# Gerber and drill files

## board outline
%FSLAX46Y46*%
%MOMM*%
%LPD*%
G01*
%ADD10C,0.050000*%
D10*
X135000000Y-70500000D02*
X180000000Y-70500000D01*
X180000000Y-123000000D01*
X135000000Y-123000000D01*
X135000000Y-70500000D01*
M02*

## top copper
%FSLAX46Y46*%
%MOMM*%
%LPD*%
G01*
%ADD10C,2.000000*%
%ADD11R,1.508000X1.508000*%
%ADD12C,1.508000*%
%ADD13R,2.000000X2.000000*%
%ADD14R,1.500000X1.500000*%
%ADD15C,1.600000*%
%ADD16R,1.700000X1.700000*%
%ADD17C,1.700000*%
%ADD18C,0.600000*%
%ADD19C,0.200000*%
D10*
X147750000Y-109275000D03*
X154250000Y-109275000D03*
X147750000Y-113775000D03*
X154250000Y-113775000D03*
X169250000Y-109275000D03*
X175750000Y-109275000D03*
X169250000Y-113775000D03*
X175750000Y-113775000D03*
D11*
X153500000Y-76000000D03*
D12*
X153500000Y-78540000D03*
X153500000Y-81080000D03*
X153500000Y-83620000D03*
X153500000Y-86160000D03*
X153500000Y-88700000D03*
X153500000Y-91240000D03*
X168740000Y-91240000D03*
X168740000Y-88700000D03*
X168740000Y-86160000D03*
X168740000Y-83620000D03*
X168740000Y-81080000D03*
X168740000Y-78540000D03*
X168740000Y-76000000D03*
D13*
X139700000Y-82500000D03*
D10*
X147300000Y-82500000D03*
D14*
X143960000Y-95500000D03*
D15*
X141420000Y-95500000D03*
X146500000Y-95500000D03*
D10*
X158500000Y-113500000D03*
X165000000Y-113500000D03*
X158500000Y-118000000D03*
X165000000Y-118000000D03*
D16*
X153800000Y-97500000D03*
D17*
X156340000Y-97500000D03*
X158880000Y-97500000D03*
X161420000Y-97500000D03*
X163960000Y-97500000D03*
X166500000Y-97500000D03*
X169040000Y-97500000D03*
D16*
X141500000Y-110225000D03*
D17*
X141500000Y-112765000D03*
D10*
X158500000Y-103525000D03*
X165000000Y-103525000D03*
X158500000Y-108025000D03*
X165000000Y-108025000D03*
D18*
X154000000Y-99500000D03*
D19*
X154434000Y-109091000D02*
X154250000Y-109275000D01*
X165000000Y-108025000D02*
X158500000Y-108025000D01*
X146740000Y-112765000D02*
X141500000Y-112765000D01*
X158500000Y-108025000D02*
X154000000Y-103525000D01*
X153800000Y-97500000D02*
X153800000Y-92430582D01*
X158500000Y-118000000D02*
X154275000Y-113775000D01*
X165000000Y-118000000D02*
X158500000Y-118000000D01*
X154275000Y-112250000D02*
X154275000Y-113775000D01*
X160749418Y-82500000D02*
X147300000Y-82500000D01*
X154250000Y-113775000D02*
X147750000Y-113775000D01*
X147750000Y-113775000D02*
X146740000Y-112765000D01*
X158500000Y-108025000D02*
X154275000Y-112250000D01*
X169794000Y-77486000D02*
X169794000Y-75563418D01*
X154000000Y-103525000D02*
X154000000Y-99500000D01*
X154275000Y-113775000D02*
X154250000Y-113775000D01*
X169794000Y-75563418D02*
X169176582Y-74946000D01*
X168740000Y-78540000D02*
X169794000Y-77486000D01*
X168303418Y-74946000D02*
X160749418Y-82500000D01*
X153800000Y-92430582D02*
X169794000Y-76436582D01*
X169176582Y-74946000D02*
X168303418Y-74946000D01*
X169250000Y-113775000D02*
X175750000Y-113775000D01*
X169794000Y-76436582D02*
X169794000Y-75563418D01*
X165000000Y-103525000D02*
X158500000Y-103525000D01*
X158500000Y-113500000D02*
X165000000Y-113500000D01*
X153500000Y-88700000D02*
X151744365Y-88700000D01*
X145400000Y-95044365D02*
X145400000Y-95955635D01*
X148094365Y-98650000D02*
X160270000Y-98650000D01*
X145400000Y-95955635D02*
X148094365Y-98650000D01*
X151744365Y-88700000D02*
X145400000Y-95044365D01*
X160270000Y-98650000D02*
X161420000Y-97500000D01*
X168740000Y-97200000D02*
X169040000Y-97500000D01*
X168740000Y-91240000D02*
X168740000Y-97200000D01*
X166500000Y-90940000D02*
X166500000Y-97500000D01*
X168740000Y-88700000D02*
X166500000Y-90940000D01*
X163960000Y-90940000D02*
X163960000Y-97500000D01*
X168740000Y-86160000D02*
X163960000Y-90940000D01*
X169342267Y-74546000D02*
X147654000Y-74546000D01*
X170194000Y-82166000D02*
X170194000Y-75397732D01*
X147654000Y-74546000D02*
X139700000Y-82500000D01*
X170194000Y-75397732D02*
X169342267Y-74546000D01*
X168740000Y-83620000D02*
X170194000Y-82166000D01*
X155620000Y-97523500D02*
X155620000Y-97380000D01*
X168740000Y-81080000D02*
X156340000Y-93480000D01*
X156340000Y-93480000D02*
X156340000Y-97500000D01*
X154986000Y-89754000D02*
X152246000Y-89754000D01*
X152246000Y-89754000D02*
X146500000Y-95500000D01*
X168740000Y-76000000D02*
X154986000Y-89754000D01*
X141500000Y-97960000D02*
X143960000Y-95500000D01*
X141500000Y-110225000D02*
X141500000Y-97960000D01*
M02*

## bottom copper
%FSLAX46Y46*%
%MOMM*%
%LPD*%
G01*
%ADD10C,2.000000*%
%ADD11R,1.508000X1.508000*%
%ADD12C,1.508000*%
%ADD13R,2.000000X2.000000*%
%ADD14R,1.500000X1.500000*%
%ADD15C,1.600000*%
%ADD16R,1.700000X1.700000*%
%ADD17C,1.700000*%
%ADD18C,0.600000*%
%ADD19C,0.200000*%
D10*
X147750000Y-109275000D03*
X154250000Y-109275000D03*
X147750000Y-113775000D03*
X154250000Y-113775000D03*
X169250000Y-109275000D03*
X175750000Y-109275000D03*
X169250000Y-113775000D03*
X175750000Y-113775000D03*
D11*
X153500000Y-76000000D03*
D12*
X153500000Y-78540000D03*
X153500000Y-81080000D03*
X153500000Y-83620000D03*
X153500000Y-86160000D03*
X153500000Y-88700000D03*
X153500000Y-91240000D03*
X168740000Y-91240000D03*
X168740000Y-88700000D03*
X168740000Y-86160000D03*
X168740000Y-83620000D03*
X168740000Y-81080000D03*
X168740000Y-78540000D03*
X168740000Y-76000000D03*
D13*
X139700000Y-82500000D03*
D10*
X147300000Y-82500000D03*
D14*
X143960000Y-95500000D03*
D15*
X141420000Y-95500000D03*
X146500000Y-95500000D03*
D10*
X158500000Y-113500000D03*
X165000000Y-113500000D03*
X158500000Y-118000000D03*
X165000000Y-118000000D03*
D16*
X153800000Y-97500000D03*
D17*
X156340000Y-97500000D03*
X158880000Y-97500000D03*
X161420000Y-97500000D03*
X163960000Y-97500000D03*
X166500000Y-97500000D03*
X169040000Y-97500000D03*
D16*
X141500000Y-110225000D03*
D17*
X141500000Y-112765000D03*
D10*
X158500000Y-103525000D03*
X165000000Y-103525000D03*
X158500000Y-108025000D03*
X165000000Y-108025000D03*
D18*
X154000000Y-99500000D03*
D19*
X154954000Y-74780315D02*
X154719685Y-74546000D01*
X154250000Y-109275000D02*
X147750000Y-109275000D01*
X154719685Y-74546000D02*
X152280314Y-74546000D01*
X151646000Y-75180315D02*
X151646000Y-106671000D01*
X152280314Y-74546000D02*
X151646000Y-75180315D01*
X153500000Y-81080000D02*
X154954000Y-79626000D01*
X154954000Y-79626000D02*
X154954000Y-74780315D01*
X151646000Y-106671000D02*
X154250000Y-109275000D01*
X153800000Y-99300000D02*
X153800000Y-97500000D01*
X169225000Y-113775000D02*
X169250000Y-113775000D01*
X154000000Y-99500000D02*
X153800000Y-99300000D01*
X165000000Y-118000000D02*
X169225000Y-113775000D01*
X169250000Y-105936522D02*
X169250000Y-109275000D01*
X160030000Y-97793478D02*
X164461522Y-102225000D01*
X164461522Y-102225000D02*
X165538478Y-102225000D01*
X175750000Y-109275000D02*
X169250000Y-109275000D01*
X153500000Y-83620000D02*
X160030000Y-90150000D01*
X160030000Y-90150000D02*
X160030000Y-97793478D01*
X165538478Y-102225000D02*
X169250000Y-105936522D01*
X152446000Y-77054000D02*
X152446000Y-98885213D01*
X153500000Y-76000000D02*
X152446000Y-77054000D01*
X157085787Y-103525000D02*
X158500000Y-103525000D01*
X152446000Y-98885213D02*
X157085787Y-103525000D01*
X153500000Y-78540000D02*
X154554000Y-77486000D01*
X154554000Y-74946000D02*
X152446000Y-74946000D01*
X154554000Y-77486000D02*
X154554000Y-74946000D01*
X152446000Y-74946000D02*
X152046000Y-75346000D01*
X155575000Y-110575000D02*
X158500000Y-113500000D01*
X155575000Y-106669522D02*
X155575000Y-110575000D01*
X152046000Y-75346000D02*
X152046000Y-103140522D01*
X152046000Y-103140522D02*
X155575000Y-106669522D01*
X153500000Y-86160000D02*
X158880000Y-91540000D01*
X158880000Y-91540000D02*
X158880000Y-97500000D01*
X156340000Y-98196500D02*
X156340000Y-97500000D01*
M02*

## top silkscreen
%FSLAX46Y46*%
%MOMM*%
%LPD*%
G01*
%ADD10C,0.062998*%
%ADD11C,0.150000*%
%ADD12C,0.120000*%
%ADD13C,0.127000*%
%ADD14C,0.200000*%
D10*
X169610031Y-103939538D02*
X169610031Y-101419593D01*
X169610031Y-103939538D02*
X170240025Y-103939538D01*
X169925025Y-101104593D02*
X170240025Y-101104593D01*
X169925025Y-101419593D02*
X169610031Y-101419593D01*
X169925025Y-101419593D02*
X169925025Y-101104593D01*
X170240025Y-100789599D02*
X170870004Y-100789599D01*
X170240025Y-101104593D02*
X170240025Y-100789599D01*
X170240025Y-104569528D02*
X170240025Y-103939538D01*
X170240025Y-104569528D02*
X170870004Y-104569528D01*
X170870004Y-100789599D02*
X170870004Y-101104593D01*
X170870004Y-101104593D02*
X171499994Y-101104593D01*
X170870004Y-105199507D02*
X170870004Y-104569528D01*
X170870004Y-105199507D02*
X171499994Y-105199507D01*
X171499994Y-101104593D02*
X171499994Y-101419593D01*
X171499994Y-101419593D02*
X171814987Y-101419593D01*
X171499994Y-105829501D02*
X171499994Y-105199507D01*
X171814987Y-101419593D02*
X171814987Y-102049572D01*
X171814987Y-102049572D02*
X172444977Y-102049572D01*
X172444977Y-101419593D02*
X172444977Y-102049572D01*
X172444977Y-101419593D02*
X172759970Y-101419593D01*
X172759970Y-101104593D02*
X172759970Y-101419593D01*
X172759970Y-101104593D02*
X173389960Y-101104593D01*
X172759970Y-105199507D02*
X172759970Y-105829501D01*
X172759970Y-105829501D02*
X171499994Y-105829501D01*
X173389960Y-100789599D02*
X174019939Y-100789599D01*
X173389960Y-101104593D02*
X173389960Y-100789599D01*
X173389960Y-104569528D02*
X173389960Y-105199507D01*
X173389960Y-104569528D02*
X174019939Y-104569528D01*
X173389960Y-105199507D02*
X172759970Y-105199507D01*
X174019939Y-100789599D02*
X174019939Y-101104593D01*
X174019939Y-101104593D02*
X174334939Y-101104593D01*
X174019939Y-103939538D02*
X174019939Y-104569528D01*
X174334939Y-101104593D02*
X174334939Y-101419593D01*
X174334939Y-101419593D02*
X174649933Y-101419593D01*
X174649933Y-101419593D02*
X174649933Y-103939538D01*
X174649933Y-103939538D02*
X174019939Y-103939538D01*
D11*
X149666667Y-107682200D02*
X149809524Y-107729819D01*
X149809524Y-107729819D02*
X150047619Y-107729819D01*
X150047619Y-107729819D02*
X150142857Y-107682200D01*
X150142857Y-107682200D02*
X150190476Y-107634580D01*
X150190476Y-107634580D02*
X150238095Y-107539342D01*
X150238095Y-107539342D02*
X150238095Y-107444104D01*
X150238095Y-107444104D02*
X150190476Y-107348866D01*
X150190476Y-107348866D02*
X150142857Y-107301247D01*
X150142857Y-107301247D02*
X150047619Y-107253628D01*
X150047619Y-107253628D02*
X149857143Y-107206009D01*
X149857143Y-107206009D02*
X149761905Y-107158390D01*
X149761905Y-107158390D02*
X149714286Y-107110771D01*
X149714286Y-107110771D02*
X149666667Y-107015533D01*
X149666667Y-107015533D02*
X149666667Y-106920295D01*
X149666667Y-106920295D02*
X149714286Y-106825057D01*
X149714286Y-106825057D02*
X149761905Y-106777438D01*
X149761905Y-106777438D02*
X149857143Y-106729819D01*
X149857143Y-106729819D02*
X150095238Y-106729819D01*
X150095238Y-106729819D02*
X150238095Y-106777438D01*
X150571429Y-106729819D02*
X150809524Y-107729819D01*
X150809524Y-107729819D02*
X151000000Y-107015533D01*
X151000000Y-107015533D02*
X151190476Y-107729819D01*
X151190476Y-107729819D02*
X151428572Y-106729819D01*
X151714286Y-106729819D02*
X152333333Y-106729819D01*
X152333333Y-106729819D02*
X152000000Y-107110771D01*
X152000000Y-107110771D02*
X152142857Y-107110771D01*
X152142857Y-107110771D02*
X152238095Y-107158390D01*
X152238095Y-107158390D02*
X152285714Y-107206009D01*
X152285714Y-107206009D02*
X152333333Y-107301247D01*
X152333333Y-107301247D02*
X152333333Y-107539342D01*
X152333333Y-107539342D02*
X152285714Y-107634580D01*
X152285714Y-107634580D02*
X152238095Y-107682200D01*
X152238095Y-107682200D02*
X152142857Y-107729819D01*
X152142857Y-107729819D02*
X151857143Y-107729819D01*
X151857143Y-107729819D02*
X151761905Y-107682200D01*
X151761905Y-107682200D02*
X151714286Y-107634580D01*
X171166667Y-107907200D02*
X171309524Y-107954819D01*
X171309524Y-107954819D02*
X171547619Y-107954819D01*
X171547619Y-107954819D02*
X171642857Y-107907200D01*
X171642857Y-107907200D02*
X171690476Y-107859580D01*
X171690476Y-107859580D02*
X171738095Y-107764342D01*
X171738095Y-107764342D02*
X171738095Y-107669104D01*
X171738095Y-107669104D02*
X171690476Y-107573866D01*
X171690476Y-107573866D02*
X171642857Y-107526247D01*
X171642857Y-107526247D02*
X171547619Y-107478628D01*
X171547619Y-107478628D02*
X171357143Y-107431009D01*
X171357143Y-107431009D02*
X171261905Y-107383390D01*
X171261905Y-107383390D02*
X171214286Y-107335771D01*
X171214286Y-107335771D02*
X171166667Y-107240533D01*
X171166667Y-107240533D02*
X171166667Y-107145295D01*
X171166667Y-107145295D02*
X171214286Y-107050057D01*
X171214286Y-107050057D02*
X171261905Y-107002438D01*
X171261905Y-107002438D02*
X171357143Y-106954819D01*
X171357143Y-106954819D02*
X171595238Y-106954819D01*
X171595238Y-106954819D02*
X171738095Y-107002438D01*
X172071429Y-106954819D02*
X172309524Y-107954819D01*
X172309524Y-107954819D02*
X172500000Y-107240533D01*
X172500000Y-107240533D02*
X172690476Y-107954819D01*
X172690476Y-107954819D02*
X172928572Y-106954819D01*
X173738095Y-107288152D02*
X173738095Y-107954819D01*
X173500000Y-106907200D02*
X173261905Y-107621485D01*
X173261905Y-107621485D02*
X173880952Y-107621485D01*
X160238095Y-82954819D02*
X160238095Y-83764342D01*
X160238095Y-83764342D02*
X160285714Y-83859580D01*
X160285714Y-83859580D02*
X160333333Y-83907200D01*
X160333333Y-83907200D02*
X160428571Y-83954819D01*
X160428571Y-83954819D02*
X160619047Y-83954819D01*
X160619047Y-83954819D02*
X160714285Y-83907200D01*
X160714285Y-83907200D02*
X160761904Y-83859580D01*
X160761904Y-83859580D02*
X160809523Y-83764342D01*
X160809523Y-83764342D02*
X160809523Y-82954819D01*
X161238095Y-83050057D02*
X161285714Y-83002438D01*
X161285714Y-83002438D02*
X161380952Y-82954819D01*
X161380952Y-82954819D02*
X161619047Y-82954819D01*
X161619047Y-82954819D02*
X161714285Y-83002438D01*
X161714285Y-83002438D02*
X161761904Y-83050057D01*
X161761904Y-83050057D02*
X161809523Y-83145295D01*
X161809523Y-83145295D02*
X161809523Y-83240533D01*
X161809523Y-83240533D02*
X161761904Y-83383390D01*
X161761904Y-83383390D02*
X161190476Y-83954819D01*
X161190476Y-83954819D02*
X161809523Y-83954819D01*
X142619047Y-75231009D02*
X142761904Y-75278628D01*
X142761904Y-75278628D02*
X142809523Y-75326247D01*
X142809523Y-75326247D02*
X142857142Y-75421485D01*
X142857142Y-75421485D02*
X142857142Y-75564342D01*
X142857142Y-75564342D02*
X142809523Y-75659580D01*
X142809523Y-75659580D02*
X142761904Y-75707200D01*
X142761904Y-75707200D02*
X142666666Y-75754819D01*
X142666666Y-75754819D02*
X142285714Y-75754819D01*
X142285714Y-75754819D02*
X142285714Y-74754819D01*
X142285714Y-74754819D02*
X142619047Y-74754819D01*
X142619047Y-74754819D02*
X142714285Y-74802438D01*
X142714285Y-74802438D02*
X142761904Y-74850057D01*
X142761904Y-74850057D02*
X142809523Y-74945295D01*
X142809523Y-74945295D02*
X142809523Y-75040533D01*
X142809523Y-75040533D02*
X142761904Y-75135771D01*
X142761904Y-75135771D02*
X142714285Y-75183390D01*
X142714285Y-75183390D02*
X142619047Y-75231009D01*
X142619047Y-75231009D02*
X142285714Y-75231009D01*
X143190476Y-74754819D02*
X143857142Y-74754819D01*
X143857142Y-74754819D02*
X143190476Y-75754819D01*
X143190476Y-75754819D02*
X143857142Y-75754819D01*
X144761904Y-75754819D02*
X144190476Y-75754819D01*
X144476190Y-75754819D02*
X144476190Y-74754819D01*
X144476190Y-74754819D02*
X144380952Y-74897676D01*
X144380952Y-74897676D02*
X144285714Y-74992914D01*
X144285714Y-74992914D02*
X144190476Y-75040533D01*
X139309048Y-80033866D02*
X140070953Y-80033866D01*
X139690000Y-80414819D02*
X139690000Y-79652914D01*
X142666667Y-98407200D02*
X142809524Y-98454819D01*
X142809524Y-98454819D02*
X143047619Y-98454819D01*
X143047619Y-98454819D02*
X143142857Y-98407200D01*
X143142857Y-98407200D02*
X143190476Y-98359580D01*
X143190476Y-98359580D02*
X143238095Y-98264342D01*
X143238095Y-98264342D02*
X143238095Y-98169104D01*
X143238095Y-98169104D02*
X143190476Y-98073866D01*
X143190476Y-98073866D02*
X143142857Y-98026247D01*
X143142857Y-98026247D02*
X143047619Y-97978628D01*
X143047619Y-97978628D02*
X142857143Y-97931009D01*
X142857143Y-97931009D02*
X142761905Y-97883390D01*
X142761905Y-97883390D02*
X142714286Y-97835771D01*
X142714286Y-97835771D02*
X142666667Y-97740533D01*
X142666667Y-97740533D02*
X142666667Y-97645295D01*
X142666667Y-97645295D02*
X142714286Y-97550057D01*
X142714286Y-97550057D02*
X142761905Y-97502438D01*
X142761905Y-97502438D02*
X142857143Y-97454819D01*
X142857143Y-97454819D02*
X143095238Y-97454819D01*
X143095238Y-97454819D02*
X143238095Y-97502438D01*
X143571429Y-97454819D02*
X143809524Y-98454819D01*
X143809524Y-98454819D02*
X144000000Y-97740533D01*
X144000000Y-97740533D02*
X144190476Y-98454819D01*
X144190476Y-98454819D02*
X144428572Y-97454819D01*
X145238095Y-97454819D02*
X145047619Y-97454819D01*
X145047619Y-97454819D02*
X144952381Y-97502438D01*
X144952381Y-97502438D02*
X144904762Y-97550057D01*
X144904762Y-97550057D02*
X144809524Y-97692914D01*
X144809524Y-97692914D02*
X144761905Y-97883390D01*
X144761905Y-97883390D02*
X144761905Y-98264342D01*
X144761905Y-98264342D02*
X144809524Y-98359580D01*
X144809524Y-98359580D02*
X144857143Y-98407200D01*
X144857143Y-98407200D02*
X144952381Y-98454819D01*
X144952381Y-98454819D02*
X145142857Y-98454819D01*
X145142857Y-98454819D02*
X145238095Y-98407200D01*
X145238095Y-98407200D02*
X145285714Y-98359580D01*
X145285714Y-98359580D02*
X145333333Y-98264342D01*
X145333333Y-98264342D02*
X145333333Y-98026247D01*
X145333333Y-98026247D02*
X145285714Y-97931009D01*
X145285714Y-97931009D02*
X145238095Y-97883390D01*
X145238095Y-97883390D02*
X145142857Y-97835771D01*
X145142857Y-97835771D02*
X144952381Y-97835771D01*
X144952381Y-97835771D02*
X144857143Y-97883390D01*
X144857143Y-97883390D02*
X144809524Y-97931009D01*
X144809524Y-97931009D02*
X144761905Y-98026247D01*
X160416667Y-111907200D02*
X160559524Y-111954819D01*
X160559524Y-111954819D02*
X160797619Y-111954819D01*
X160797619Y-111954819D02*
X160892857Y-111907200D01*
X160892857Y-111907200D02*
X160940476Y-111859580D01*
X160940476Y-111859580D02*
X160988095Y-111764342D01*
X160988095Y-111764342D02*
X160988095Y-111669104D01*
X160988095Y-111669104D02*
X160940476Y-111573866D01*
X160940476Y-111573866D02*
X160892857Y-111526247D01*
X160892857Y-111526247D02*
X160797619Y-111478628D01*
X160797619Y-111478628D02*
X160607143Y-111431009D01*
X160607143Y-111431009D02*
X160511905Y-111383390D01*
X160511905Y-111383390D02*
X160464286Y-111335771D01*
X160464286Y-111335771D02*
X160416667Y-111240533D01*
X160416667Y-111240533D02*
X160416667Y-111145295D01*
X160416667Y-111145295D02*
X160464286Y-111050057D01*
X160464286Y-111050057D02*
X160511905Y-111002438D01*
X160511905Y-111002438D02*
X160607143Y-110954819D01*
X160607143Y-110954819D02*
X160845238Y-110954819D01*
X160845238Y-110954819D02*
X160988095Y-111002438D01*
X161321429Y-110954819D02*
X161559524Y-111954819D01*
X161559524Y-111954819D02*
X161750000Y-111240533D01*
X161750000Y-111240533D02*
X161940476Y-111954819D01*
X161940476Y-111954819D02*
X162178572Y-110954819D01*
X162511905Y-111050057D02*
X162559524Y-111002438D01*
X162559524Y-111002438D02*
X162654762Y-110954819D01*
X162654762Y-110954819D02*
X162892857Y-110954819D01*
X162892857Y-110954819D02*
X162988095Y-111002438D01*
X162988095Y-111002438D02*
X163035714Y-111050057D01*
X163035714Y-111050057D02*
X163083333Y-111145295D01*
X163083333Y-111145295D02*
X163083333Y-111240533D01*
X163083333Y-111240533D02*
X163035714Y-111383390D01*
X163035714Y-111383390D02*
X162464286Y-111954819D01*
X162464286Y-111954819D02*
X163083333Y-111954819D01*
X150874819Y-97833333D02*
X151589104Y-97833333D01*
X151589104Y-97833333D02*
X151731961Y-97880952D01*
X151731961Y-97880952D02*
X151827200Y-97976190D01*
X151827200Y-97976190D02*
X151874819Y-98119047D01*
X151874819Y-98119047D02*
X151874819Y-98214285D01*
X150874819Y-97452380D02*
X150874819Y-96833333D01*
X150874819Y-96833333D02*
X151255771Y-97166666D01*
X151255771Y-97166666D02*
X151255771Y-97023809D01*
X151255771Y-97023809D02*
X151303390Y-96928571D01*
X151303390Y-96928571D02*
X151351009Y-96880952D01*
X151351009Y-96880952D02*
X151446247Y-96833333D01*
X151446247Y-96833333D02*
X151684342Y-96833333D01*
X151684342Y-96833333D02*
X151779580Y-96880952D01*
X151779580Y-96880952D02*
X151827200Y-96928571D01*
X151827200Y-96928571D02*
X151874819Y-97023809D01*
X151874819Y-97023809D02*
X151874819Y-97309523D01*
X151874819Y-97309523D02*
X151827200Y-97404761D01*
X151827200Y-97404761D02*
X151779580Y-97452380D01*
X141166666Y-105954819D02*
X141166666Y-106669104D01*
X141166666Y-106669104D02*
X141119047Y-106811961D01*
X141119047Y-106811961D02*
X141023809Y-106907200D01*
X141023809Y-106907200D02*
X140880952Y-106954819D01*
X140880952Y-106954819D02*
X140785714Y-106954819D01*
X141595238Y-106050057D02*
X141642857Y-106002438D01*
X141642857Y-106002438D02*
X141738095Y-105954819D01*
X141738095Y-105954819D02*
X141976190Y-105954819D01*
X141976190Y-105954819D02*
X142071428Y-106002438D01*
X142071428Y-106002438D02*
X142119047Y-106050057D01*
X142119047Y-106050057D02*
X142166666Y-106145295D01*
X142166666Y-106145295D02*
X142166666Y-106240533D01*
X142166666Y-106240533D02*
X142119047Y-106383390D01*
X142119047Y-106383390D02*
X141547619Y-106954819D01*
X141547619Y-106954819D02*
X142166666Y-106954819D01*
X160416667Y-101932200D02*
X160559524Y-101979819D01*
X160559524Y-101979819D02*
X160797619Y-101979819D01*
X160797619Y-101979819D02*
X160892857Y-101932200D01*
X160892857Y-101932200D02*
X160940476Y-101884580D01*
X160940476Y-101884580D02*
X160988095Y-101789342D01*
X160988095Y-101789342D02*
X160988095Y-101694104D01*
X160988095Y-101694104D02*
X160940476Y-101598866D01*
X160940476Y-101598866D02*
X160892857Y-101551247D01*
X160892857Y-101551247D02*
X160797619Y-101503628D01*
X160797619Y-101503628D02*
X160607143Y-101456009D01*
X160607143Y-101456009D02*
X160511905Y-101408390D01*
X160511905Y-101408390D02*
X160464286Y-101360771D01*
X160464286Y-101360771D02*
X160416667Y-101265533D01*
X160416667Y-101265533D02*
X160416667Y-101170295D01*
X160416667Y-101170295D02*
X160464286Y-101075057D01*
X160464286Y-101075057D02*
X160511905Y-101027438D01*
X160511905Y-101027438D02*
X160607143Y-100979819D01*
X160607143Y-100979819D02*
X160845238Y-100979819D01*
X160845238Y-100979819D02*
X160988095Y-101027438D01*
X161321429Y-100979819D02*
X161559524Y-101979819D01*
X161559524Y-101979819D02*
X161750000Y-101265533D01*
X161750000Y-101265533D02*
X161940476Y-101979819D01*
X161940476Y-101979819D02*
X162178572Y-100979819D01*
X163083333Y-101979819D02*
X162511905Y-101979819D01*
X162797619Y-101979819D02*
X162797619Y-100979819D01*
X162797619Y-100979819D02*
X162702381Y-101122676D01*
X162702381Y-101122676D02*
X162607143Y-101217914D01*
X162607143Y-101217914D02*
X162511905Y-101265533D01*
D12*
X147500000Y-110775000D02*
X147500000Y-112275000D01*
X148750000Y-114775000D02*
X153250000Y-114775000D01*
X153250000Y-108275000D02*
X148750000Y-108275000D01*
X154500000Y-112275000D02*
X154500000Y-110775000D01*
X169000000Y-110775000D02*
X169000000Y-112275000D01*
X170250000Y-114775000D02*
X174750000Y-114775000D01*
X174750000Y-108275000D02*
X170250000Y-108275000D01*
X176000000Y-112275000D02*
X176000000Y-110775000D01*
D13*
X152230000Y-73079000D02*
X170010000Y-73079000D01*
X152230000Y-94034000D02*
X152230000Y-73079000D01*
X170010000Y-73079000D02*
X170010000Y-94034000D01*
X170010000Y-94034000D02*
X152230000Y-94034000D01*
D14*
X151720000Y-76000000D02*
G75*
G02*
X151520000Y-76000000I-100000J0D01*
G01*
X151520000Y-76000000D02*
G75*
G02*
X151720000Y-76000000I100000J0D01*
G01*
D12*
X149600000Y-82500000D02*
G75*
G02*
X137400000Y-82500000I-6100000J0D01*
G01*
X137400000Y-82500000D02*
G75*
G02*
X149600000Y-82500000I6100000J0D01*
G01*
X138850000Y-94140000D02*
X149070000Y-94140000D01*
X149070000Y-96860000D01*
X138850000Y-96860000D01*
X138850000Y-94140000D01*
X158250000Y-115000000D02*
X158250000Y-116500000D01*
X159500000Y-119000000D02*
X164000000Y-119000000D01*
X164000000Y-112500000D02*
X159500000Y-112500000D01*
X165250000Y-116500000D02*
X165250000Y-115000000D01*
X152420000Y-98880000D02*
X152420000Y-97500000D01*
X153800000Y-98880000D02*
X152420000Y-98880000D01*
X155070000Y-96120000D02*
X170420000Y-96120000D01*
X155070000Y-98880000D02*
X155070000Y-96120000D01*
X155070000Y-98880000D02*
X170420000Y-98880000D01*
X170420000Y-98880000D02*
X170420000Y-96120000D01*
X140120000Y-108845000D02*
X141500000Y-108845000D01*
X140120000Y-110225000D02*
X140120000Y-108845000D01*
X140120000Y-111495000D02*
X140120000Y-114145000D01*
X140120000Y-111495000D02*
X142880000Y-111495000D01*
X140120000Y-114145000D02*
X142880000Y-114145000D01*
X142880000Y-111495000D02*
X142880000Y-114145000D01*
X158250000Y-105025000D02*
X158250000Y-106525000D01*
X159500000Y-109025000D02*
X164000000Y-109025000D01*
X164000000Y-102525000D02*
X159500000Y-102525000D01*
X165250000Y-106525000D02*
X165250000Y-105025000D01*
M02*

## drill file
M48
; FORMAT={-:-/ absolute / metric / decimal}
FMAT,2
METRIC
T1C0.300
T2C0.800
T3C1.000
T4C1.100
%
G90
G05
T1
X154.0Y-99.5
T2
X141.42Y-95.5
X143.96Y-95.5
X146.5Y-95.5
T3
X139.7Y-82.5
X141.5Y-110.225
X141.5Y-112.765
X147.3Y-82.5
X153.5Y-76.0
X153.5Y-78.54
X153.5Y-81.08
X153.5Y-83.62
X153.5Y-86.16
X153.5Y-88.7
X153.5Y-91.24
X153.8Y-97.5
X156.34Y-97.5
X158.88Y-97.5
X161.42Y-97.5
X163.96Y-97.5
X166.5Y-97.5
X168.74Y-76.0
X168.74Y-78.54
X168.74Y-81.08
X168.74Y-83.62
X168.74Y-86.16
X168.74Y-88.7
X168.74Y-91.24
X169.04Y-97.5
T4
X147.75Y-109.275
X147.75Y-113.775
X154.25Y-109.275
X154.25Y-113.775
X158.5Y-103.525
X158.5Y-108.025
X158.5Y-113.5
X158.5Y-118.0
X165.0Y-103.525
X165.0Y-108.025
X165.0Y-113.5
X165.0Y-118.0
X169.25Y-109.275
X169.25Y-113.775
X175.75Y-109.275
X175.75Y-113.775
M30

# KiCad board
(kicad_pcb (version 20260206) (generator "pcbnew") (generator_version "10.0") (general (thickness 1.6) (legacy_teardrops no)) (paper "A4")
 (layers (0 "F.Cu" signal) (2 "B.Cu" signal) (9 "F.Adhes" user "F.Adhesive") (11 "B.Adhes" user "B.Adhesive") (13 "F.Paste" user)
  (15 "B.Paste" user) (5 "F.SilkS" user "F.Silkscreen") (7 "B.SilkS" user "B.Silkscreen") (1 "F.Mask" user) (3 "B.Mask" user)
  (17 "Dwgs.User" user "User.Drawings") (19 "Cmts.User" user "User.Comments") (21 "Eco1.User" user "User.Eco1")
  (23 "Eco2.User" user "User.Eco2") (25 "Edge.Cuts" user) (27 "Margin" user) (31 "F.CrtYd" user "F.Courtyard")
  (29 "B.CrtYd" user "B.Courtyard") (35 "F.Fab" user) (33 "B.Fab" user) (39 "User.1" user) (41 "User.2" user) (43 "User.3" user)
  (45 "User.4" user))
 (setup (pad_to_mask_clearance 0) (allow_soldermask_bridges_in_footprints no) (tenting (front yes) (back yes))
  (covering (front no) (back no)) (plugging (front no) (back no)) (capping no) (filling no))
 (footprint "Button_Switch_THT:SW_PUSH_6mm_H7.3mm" (layer "F.Cu") (at 147.75 109.275)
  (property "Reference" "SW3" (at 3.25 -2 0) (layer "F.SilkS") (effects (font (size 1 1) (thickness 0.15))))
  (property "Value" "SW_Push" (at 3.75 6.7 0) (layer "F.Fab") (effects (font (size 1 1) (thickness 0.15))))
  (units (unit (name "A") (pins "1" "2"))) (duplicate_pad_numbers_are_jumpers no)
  (fp_line (start -0.25 1.5) (end -0.25 3) (stroke (width 0.12) (type solid)) (layer "F.SilkS"))
  (fp_line (start 1 5.5) (end 5.5 5.5) (stroke (width 0.12) (type solid)) (layer "F.SilkS"))
  (fp_line (start 5.5 -1) (end 1 -1) (stroke (width 0.12) (type solid)) (layer "F.SilkS"))
  (fp_line (start 6.75 3) (end 6.75 1.5) (stroke (width 0.12) (type solid)) (layer "F.SilkS"))
  (pad "1" thru_hole circle (at 0 0 90) (size 2 2) (drill 1.1) (layers "*.Cu" "*.Mask") (remove_unused_layers no) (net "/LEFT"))
  (pad "1" thru_hole circle (at 6.5 0 90) (size 2 2) (drill 1.1) (layers "*.Cu" "*.Mask") (remove_unused_layers no) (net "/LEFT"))
  (pad "2" thru_hole circle (at 0 4.5 90) (size 2 2) (drill 1.1) (layers "*.Cu" "*.Mask") (remove_unused_layers no) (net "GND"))
  (pad "2" thru_hole circle (at 6.5 4.5 90) (size 2 2) (drill 1.1) (layers "*.Cu" "*.Mask") (remove_unused_layers no) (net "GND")))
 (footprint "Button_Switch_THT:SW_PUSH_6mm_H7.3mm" (layer "F.Cu") (at 169.25 109.275)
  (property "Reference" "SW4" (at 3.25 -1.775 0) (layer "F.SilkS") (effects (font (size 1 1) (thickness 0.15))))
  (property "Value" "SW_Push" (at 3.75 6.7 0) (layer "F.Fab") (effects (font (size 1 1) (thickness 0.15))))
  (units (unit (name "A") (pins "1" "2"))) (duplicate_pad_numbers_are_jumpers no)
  (fp_line (start -0.25 1.5) (end -0.25 3) (stroke (width 0.12) (type solid)) (layer "F.SilkS"))
  (fp_line (start 1 5.5) (end 5.5 5.5) (stroke (width 0.12) (type solid)) (layer "F.SilkS"))
  (fp_line (start 5.5 -1) (end 1 -1) (stroke (width 0.12) (type solid)) (layer "F.SilkS"))
  (fp_line (start 6.75 3) (end 6.75 1.5) (stroke (width 0.12) (type solid)) (layer "F.SilkS"))
  (pad "1" thru_hole circle (at 0 0 90) (size 2 2) (drill 1.1) (layers "*.Cu" "*.Mask") (remove_unused_layers no) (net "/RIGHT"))
  (pad "1" thru_hole circle (at 6.5 0 90) (size 2 2) (drill 1.1) (layers "*.Cu" "*.Mask") (remove_unused_layers no) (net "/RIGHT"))
  (pad "2" thru_hole circle (at 0 4.5 90) (size 2 2) (drill 1.1) (layers "*.Cu" "*.Mask") (remove_unused_layers no) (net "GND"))
  (pad "2" thru_hole circle (at 6.5 4.5 90) (size 2 2) (drill 1.1) (layers "*.Cu" "*.Mask") (remove_unused_layers no) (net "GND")))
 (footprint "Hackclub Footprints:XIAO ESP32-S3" (layer "F.Cu") (at 161.12 83.5565)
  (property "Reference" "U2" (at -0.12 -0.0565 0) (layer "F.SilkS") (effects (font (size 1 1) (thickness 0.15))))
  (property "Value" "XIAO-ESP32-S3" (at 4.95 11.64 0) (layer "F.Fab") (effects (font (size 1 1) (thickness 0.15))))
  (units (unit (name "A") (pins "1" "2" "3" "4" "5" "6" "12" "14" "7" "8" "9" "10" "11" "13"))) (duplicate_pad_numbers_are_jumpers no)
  (fp_line (start -8.89 -10.4775) (end 8.89 -10.4775) (stroke (width 0.127) (type solid)) (layer "F.SilkS"))
  (fp_line (start -8.89 10.4775) (end -8.89 -10.4775) (stroke (width 0.127) (type solid)) (layer "F.SilkS"))
  (fp_line (start 8.89 -10.4775) (end 8.89 10.4775) (stroke (width 0.127) (type solid)) (layer "F.SilkS"))
  (fp_line (start 8.89 10.4775) (end -8.89 10.4775) (stroke (width 0.127) (type solid)) (layer "F.SilkS"))
  (fp_circle (center -9.5 -7.5565) (end -9.4 -7.5565) (stroke (width 0.2) (type solid)) (fill no) (layer "F.SilkS"))
  (pad "1" thru_hole rect (at -7.62 -7.5565) (size 1.508 1.508) (drill 1) (layers "*.Cu" "*.Mask") (remove_unused_layers no) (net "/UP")
   (solder_mask_margin 0.102))
  (pad "2" thru_hole circle (at -7.62 -5.0165) (size 1.508 1.508) (drill 1) (layers "*.Cu" "*.Mask") (remove_unused_layers no) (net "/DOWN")
   (solder_mask_margin 0.102))
  (pad "3" thru_hole circle (at -7.62 -2.4765) (size 1.508 1.508) (drill 1) (layers "*.Cu" "*.Mask") (remove_unused_layers no) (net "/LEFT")
   (solder_mask_margin 0.102))
  (pad "4" thru_hole circle (at -7.62 0.0635) (size 1.508 1.508) (drill 1) (layers "*.Cu" "*.Mask") (remove_unused_layers no) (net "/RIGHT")
   (solder_mask_margin 0.102))
  (pad "5" thru_hole circle (at -7.62 2.6035) (size 1.508 1.508) (drill 1) (layers "*.Cu" "*.Mask") (remove_unused_layers no) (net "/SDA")
   (solder_mask_margin 0.102))
  (pad "6" thru_hole circle (at -7.62 5.1435) (size 1.508 1.508) (drill 1) (layers "*.Cu" "*.Mask") (remove_unused_layers no) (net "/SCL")
   (solder_mask_margin 0.102))
  (pad "7" thru_hole circle (at -7.62 7.6835) (size 1.508 1.508) (drill 1) (layers "*.Cu" "*.Mask") (remove_unused_layers no)
   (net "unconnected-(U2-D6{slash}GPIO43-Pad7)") (solder_mask_margin 0.102))
  (pad "8" thru_hole circle (at 7.62 7.6835) (size 1.508 1.508) (drill 1) (layers "*.Cu" "*.Mask") (remove_unused_layers no)
   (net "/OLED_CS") (solder_mask_margin 0.102))
  (pad "9" thru_hole circle (at 7.62 5.1435) (size 1.508 1.508) (drill 1) (layers "*.Cu" "*.Mask") (remove_unused_layers no)
   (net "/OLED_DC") (solder_mask_margin 0.102))
  (pad "10" thru_hole circle (at 7.62 2.6035) (size 1.508 1.508) (drill 1) (layers "*.Cu" "*.Mask") (remove_unused_layers no)
   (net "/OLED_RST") (solder_mask_margin 0.102))
  (pad "11" thru_hole circle (at 7.62 0.0635) (size 1.508 1.508) (drill 1) (layers "*.Cu" "*.Mask") (remove_unused_layers no)
   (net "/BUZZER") (solder_mask_margin 0.102))
  (pad "12" thru_hole circle (at 7.62 -2.4765) (size 1.508 1.508) (drill 1) (layers "*.Cu" "*.Mask") (remove_unused_layers no) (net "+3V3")
   (solder_mask_margin 0.102))
  (pad "13" thru_hole circle (at 7.62 -5.0165) (size 1.508 1.508) (drill 1) (layers "*.Cu" "*.Mask") (remove_unused_layers no) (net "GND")
   (solder_mask_margin 0.102))
  (pad "14" thru_hole circle (at 7.62 -7.5565) (size 1.508 1.508) (drill 1) (layers "*.Cu" "*.Mask") (remove_unused_layers no) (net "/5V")
   (solder_mask_margin 0.102)))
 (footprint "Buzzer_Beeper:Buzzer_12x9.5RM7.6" (layer "F.Cu") (at 139.7 82.5)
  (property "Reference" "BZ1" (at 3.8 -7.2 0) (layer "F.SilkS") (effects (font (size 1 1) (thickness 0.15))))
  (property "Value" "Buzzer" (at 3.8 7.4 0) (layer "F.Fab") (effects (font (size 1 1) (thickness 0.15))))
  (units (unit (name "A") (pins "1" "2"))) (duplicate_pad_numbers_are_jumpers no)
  (fp_circle (center 3.8 0) (end 9.9 0) (stroke (width 0.12) (type solid)) (fill no) (layer "F.SilkS"))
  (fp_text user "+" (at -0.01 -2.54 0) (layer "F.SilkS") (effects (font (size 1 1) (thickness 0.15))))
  (pad "1" thru_hole rect (at 0 0) (size 2 2) (drill 1) (layers "*.Cu" "*.Mask") (remove_unused_layers no) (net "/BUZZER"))
  (pad "2" thru_hole circle (at 7.6 0) (size 2 2) (drill 1) (layers "*.Cu" "*.Mask") (remove_unused_layers no) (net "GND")))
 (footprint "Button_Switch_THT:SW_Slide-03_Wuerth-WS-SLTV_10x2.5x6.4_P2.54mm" (layer "F.Cu") (at 143.96 95.5)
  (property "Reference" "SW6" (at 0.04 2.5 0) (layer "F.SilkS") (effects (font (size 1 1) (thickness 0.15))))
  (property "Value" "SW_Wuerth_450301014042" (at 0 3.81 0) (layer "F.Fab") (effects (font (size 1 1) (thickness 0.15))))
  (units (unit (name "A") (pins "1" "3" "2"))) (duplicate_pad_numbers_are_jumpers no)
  (fp_rect (start -5.11 -1.36) (end 5.11 1.36) (stroke (width 0.12) (type default)) (fill no) (layer "F.SilkS"))
  (pad "1" thru_hole rect (at 0 0) (size 1.5 1.5) (drill 0.8) (layers "*.Cu" "*.Mask") (remove_unused_layers no) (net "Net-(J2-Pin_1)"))
  (pad "2" thru_hole circle (at -2.54 0) (size 1.6 1.6) (drill 0.8) (layers "*.Cu" "*.Mask") (remove_unused_layers no)
   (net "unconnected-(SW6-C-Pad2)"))
  (pad "3" thru_hole circle (at 2.54 0) (size 1.6 1.6) (drill 0.8) (layers "*.Cu" "*.Mask") (remove_unused_layers no) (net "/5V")))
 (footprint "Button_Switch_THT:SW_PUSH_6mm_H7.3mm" (layer "F.Cu") (at 158.5 113.5)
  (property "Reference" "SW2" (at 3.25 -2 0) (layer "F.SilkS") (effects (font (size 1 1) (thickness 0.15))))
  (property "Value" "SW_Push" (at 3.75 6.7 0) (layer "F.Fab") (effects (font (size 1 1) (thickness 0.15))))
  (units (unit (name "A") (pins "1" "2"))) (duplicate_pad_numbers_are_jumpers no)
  (fp_line (start -0.25 1.5) (end -0.25 3) (stroke (width 0.12) (type solid)) (layer "F.SilkS"))
  (fp_line (start 1 5.5) (end 5.5 5.5) (stroke (width 0.12) (type solid)) (layer "F.SilkS"))
  (fp_line (start 5.5 -1) (end 1 -1) (stroke (width 0.12) (type solid)) (layer "F.SilkS"))
  (fp_line (start 6.75 3) (end 6.75 1.5) (stroke (width 0.12) (type solid)) (layer "F.SilkS"))
  (pad "1" thru_hole circle (at 0 0 90) (size 2 2) (drill 1.1) (layers "*.Cu" "*.Mask") (remove_unused_layers no) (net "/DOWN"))
  (pad "1" thru_hole circle (at 6.5 0 90) (size 2 2) (drill 1.1) (layers "*.Cu" "*.Mask") (remove_unused_layers no) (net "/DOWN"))
  (pad "2" thru_hole circle (at 0 4.5 90) (size 2 2) (drill 1.1) (layers "*.Cu" "*.Mask") (remove_unused_layers no) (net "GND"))
  (pad "2" thru_hole circle (at 6.5 4.5 90) (size 2 2) (drill 1.1) (layers "*.Cu" "*.Mask") (remove_unused_layers no) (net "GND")))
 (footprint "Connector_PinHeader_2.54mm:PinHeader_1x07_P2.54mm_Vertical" (layer "F.Cu") (at 153.8 97.5 90)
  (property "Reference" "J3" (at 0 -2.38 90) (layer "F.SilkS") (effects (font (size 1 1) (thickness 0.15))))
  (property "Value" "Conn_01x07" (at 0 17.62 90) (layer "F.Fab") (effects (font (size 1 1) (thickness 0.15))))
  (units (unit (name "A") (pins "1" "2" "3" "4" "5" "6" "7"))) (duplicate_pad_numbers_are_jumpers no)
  (fp_line (start -1.38 -1.38) (end 0 -1.38) (stroke (width 0.12) (type solid)) (layer "F.SilkS"))
  (fp_line (start -1.38 0) (end -1.38 -1.38) (stroke (width 0.12) (type solid)) (layer "F.SilkS"))
  (fp_line (start 1.38 1.27) (end 1.38 16.62) (stroke (width 0.12) (type solid)) (layer "F.SilkS"))
  (fp_line (start -1.38 1.27) (end 1.38 1.27) (stroke (width 0.12) (type solid)) (layer "F.SilkS"))
  (fp_line (start -1.38 1.27) (end -1.38 16.62) (stroke (width 0.12) (type solid)) (layer "F.SilkS"))
  (fp_line (start -1.38 16.62) (end 1.38 16.62) (stroke (width 0.12) (type solid)) (layer "F.SilkS"))
  (pad "1" thru_hole rect (at 0 0 90) (size 1.7 1.7) (drill 1) (layers "*.Cu" "*.Mask") (remove_unused_layers no) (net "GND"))
  (pad "2" thru_hole circle (at 0 2.54 90) (size 1.7 1.7) (drill 1) (layers "*.Cu" "*.Mask") (remove_unused_layers no) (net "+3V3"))
  (pad "3" thru_hole circle (at 0 5.08 90) (size 1.7 1.7) (drill 1) (layers "*.Cu" "*.Mask") (remove_unused_layers no) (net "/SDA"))
  (pad "4" thru_hole circle (at 0 7.62 90) (size 1.7 1.7) (drill 1) (layers "*.Cu" "*.Mask") (remove_unused_layers no) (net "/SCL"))
  (pad "5" thru_hole circle (at 0 10.16 90) (size 1.7 1.7) (drill 1) (layers "*.Cu" "*.Mask") (remove_unused_layers no) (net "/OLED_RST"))
  (pad "6" thru_hole circle (at 0 12.7 90) (size 1.7 1.7) (drill 1) (layers "*.Cu" "*.Mask") (remove_unused_layers no) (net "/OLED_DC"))
  (pad "7" thru_hole circle (at 0 15.24 90) (size 1.7 1.7) (drill 1) (layers "*.Cu" "*.Mask") (remove_unused_layers no) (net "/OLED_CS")))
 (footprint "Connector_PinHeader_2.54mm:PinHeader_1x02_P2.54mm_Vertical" (layer "F.Cu") (at 141.5 110.225)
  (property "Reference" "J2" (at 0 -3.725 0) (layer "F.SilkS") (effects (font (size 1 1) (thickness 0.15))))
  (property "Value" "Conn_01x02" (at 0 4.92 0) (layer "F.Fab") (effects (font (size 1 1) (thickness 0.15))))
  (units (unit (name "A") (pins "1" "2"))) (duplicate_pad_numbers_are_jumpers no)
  (fp_line (start -1.38 -1.38) (end 0 -1.38) (stroke (width 0.12) (type solid)) (layer "F.SilkS"))
  (fp_line (start -1.38 0) (end -1.38 -1.38) (stroke (width 0.12) (type solid)) (layer "F.SilkS"))
  (fp_line (start -1.38 1.27) (end -1.38 3.92) (stroke (width 0.12) (type solid)) (layer "F.SilkS"))
  (fp_line (start -1.38 1.27) (end 1.38 1.27) (stroke (width 0.12) (type solid)) (layer "F.SilkS"))
  (fp_line (start -1.38 3.92) (end 1.38 3.92) (stroke (width 0.12) (type solid)) (layer "F.SilkS"))
  (fp_line (start 1.38 1.27) (end 1.38 3.92) (stroke (width 0.12) (type solid)) (layer "F.SilkS"))
  (pad "1" thru_hole rect (at 0 0) (size 1.7 1.7) (drill 1) (layers "*.Cu" "*.Mask") (remove_unused_layers no) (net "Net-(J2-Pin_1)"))
  (pad "2" thru_hole circle (at 0 2.54) (size 1.7 1.7) (drill 1) (layers "*.Cu" "*.Mask") (remove_unused_layers no) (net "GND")))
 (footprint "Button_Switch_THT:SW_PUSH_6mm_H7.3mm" (layer "F.Cu") (at 158.5 103.525)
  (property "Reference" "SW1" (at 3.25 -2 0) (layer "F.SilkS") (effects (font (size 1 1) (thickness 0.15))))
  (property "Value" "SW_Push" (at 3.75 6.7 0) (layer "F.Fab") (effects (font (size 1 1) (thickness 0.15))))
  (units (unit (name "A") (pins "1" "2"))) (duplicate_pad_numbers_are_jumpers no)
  (fp_line (start -0.25 1.5) (end -0.25 3) (stroke (width 0.12) (type solid)) (layer "F.SilkS"))
  (fp_line (start 1 5.5) (end 5.5 5.5) (stroke (width 0.12) (type solid)) (layer "F.SilkS"))
  (fp_line (start 5.5 -1) (end 1 -1) (stroke (width 0.12) (type solid)) (layer "F.SilkS"))
  (fp_line (start 6.75 3) (end 6.75 1.5) (stroke (width 0.12) (type solid)) (layer "F.SilkS"))
  (pad "1" thru_hole circle (at 0 0 90) (size 2 2) (drill 1.1) (layers "*.Cu" "*.Mask") (remove_unused_layers no) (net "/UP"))
  (pad "1" thru_hole circle (at 6.5 0 90) (size 2 2) (drill 1.1) (layers "*.Cu" "*.Mask") (remove_unused_layers no) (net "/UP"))
  (pad "2" thru_hole circle (at 0 4.5 90) (size 2 2) (drill 1.1) (layers "*.Cu" "*.Mask") (remove_unused_layers no) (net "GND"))
  (pad "2" thru_hole circle (at 6.5 4.5 90) (size 2 2) (drill 1.1) (layers "*.Cu" "*.Mask") (remove_unused_layers no) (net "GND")))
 (gr_line (start 169.610031 103.939538) (end 169.610031 101.419593) (stroke (width 0.062998) (type default)) (layer "F.SilkS"))
 (gr_line (start 169.610031 103.939538) (end 170.240025 103.939538) (stroke (width 0.062998) (type default)) (layer "F.SilkS"))
 (gr_line (start 169.925025 101.104593) (end 170.240025 101.104593) (stroke (width 0.062998) (type default)) (layer "F.SilkS"))
 (gr_line (start 169.925025 101.419593) (end 169.610031 101.419593) (stroke (width 0.062998) (type default)) (layer "F.SilkS"))
 (gr_line (start 169.925025 101.419593) (end 169.925025 101.104593) (stroke (width 0.062998) (type default)) (layer "F.SilkS"))
 (gr_line (start 170.240025 100.789599) (end 170.870004 100.789599) (stroke (width 0.062998) (type default)) (layer "F.SilkS"))
 (gr_line (start 170.240025 101.104593) (end 170.240025 100.789599) (stroke (width 0.062998) (type default)) (layer "F.SilkS"))
 (gr_line (start 170.240025 104.569528) (end 170.240025 103.939538) (stroke (width 0.062998) (type default)) (layer "F.SilkS"))
 (gr_line (start 170.240025 104.569528) (end 170.870004 104.569528) (stroke (width 0.062998) (type default)) (layer "F.SilkS"))
 (gr_line (start 170.870004 100.789599) (end 170.870004 101.104593) (stroke (width 0.062998) (type default)) (layer "F.SilkS"))
 (gr_line (start 170.870004 101.104593) (end 171.499994 101.104593) (stroke (width 0.062998) (type default)) (layer "F.SilkS"))
 (gr_line (start 170.870004 105.199507) (end 170.870004 104.569528) (stroke (width 0.062998) (type default)) (layer "F.SilkS"))
 (gr_line (start 170.870004 105.199507) (end 171.499994 105.199507) (stroke (width 0.062998) (type default)) (layer "F.SilkS"))
 (gr_line (start 171.499994 101.104593) (end 171.499994 101.419593) (stroke (width 0.062998) (type default)) (layer "F.SilkS"))
 (gr_line (start 171.499994 101.419593) (end 171.814987 101.419593) (stroke (width 0.062998) (type default)) (layer "F.SilkS"))
 (gr_line (start 171.499994 105.829501) (end 171.499994 105.199507) (stroke (width 0.062998) (type default)) (layer "F.SilkS"))
 (gr_line (start 171.814987 101.419593) (end 171.814987 102.049572) (stroke (width 0.062998) (type default)) (layer "F.SilkS"))
 (gr_line (start 171.814987 102.049572) (end 172.444977 102.049572) (stroke (width 0.062998) (type default)) (layer "F.SilkS"))
 (gr_line (start 172.444977 101.419593) (end 172.444977 102.049572) (stroke (width 0.062998) (type default)) (layer "F.SilkS"))
 (gr_line (start 172.444977 101.419593) (end 172.75997 101.419593) (stroke (width 0.062998) (type default)) (layer "F.SilkS"))
 (gr_line (start 172.75997 101.104593) (end 172.75997 101.419593) (stroke (width 0.062998) (type default)) (layer "F.SilkS"))
 (gr_line (start 172.75997 101.104593) (end 173.38996 101.104593) (stroke (width 0.062998) (type default)) (layer "F.SilkS"))
 (gr_line (start 172.75997 105.199507) (end 172.75997 105.829501) (stroke (width 0.062998) (type default)) (layer "F.SilkS"))
 (gr_line (start 172.75997 105.829501) (end 171.499994 105.829501) (stroke (width 0.062998) (type default)) (layer "F.SilkS"))
 (gr_line (start 173.38996 100.789599) (end 174.019939 100.789599) (stroke (width 0.062998) (type default)) (layer "F.SilkS"))
 (gr_line (start 173.38996 101.104593) (end 173.38996 100.789599) (stroke (width 0.062998) (type default)) (layer "F.SilkS"))
 (gr_line (start 173.38996 104.569528) (end 173.38996 105.199507) (stroke (width 0.062998) (type default)) (layer "F.SilkS"))
 (gr_line (start 173.38996 104.569528) (end 174.019939 104.569528) (stroke (width 0.062998) (type default)) (layer "F.SilkS"))
 (gr_line (start 173.38996 105.199507) (end 172.75997 105.199507) (stroke (width 0.062998) (type default)) (layer "F.SilkS"))
 (gr_line (start 174.019939 100.789599) (end 174.019939 101.104593) (stroke (width 0.062998) (type default)) (layer "F.SilkS"))
 (gr_line (start 174.019939 101.104593) (end 174.334939 101.104593) (stroke (width 0.062998) (type default)) (layer "F.SilkS"))
 (gr_line (start 174.019939 103.939538) (end 174.019939 104.569528) (stroke (width 0.062998) (type default)) (layer "F.SilkS"))
 (gr_line (start 174.334939 101.104593) (end 174.334939 101.419593) (stroke (width 0.062998) (type default)) (layer "F.SilkS"))
 (gr_line (start 174.334939 101.419593) (end 174.649933 101.419593) (stroke (width 0.062998) (type default)) (layer "F.SilkS"))
 (gr_line (start 174.649933 101.419593) (end 174.649933 103.939538) (stroke (width 0.062998) (type default)) (layer "F.SilkS"))
 (gr_line (start 174.649933 103.939538) (end 174.019939 103.939538) (stroke (width 0.062998) (type default)) (layer "F.SilkS"))
 (gr_rect (start 135 70.5) (end 180 123) (stroke (width 0.05) (type default)) (fill no) (layer "Edge.Cuts"))
 (segment (start 154.434 109.091) (end 154.25 109.275) (width 0.2) (layer "F.Cu") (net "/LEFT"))
 (segment (start 154.954 74.780315) (end 154.719685 74.546) (width 0.2) (layer "B.Cu") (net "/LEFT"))
 (segment (start 154.25 109.275) (end 147.75 109.275) (width 0.2) (layer "B.Cu") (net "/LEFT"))
 (segment (start 154.719685 74.546) (end 152.280314 74.546) (width 0.2) (layer "B.Cu") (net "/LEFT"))
 (segment (start 151.646 75.180315) (end 151.646 106.671) (width 0.2) (layer "B.Cu") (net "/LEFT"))
 (segment (start 152.280314 74.546) (end 151.646 75.180315) (width 0.2) (layer "B.Cu") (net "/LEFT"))
 (segment (start 153.5 81.08) (end 154.954 79.626) (width 0.2) (layer "B.Cu") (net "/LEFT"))
 (segment (start 154.954 79.626) (end 154.954 74.780315) (width 0.2) (layer "B.Cu") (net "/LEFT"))
 (segment (start 151.646 106.671) (end 154.25 109.275) (width 0.2) (layer "B.Cu") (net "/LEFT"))
 (segment (start 165 108.025) (end 158.5 108.025) (width 0.2) (layer "F.Cu") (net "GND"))
 (segment (start 146.74 112.765) (end 141.5 112.765) (width 0.2) (layer "F.Cu") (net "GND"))
 (segment (start 158.5 108.025) (end 154 103.525) (width 0.2) (layer "F.Cu") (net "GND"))
 (segment (start 153.8 97.5) (end 153.8 92.430582) (width 0.2) (layer "F.Cu") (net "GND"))
 (segment (start 158.5 118) (end 154.275 113.775) (width 0.2) (layer "F.Cu") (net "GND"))
 (segment (start 165 118) (end 158.5 118) (width 0.2) (layer "F.Cu") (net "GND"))
 (segment (start 154.275 112.25) (end 154.275 113.775) (width 0.2) (layer "F.Cu") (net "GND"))
 (segment (start 160.749418 82.5) (end 147.3 82.5) (width 0.2) (layer "F.Cu") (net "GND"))
 (segment (start 154.25 113.775) (end 147.75 113.775) (width 0.2) (layer "F.Cu") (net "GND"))
 (segment (start 147.75 113.775) (end 146.74 112.765) (width 0.2) (layer "F.Cu") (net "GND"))
 (segment (start 158.5 108.025) (end 154.275 112.25) (width 0.2) (layer "F.Cu") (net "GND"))
 (segment (start 169.794 77.486) (end 169.794 75.563418) (width 0.2) (layer "F.Cu") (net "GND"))
 (segment (start 154 103.525) (end 154 99.5) (width 0.2) (layer "F.Cu") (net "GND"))
 (segment (start 154.275 113.775) (end 154.25 113.775) (width 0.2) (layer "F.Cu") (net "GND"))
 (segment (start 169.794 75.563418) (end 169.176582 74.946) (width 0.2) (layer "F.Cu") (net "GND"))
 (segment (start 168.74 78.54) (end 169.794 77.486) (width 0.2) (layer "F.Cu") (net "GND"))
 (segment (start 168.303418 74.946) (end 160.749418 82.5) (width 0.2) (layer "F.Cu") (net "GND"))
 (segment (start 153.8 92.430582) (end 169.794 76.436582) (width 0.2) (layer "F.Cu") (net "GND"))
 (segment (start 169.176582 74.946) (end 168.303418 74.946) (width 0.2) (layer "F.Cu") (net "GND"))
 (segment (start 169.25 113.775) (end 175.75 113.775) (width 0.2) (layer "F.Cu") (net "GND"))
 (segment (start 169.794 76.436582) (end 169.794 75.563418) (width 0.2) (layer "F.Cu") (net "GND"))
 (via (at 154 99.5) (size 0.6) (drill 0.3) (layers "F.Cu" "B.Cu") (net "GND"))
 (segment (start 153.8 99.3) (end 153.8 97.5) (width 0.2) (layer "B.Cu") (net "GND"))
 (segment (start 169.225 113.775) (end 169.25 113.775) (width 0.2) (layer "B.Cu") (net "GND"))
 (segment (start 154 99.5) (end 153.8 99.3) (width 0.2) (layer "B.Cu") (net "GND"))
 (segment (start 165 118) (end 169.225 113.775) (width 0.2) (layer "B.Cu") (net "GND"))
 (segment (start 169.25 105.936522) (end 169.25 109.275) (width 0.2) (layer "B.Cu") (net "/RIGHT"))
 (segment (start 160.03 97.793478) (end 164.461522 102.225) (width 0.2) (layer "B.Cu") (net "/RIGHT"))
 (segment (start 164.461522 102.225) (end 165.538478 102.225) (width 0.2) (layer "B.Cu") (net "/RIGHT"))
 (segment (start 175.75 109.275) (end 169.25 109.275) (width 0.2) (layer "B.Cu") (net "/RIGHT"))
 (segment (start 153.5 83.62) (end 160.03 90.15) (width 0.2) (layer "B.Cu") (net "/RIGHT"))
 (segment (start 160.03 90.15) (end 160.03 97.793478) (width 0.2) (layer "B.Cu") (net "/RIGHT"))
 (segment (start 165.538478 102.225) (end 169.25 105.936522) (width 0.2) (layer "B.Cu") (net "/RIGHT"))
 (segment (start 165 103.525) (end 158.5 103.525) (width 0.2) (layer "F.Cu") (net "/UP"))
 (segment (start 152.446 77.054) (end 152.446 98.885213) (width 0.2) (layer "B.Cu") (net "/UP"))
 (segment (start 153.5 76) (end 152.446 77.054) (width 0.2) (layer "B.Cu") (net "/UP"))
 (segment (start 157.085787 103.525) (end 158.5 103.525) (width 0.2) (layer "B.Cu") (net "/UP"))
 (segment (start 152.446 98.885213) (end 157.085787 103.525) (width 0.2) (layer "B.Cu") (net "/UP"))
 (segment (start 158.5 113.5) (end 165 113.5) (width 0.2) (layer "F.Cu") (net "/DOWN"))
 (segment (start 153.5 78.54) (end 154.554 77.486) (width 0.2) (layer "B.Cu") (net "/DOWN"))
 (segment (start 154.554 74.946) (end 152.446 74.946) (width 0.2) (layer "B.Cu") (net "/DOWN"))
 (segment (start 154.554 77.486) (end 154.554 74.946) (width 0.2) (layer "B.Cu") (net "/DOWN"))
 (segment (start 152.446 74.946) (end 152.046 75.346) (width 0.2) (layer "B.Cu") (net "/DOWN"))
 (segment (start 155.575 110.575) (end 158.5 113.5) (width 0.2) (layer "B.Cu") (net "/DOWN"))
 (segment (start 155.575 106.669522) (end 155.575 110.575) (width 0.2) (layer "B.Cu") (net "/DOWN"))
 (segment (start 152.046 75.346) (end 152.046 103.140522) (width 0.2) (layer "B.Cu") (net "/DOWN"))
 (segment (start 152.046 103.140522) (end 155.575 106.669522) (width 0.2) (layer "B.Cu") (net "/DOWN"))
 (segment (start 153.5 86.16) (end 158.88 91.54) (width 0.2) (layer "B.Cu") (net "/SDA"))
 (segment (start 158.88 91.54) (end 158.88 97.5) (width 0.2) (layer "B.Cu") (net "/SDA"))
 (segment (start 153.5 88.7) (end 151.744365 88.7) (width 0.2) (layer "F.Cu") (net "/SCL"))
 (segment (start 145.4 95.044365) (end 145.4 95.955635) (width 0.2) (layer "F.Cu") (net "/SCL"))
 (segment (start 148.094365 98.65) (end 160.27 98.65) (width 0.2) (layer "F.Cu") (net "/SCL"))
 (segment (start 145.4 95.955635) (end 148.094365 98.65) (width 0.2) (layer "F.Cu") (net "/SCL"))
 (segment (start 151.744365 88.7) (end 145.4 95.044365) (width 0.2) (layer "F.Cu") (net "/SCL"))
 (segment (start 160.27 98.65) (end 161.42 97.5) (width 0.2) (layer "F.Cu") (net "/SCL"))
 (segment (start 168.74 97.2) (end 169.04 97.5) (width 0.2) (layer "F.Cu") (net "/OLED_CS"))
 (segment (start 168.74 91.24) (end 168.74 97.2) (width 0.2) (layer "F.Cu") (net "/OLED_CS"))
 (segment (start 166.5 90.94) (end 166.5 97.5) (width 0.2) (layer "F.Cu") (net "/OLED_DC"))
 (segment (start 168.74 88.7) (end 166.5 90.94) (width 0.2) (layer "F.Cu") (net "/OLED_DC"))
 (segment (start 163.96 90.94) (end 163.96 97.5) (width 0.2) (layer "F.Cu") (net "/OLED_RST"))
 (segment (start 168.74 86.16) (end 163.96 90.94) (width 0.2) (layer "F.Cu") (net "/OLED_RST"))
 (segment (start 169.342267 74.546) (end 147.654 74.546) (width 0.2) (layer "F.Cu") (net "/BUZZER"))
 (segment (start 170.194 82.166) (end 170.194 75.397732) (width 0.2) (layer "F.Cu") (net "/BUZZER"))
 (segment (start 147.654 74.546) (end 139.7 82.5) (width 0.2) (layer "F.Cu") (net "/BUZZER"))
 (segment (start 170.194 75.397732) (end 169.342267 74.546) (width 0.2) (layer "F.Cu") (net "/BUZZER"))
 (segment (start 168.74 83.62) (end 170.194 82.166) (width 0.2) (layer "F.Cu") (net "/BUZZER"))
 (segment (start 155.62 97.5235) (end 155.62 97.38) (width 0.2) (layer "F.Cu") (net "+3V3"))
 (segment (start 168.74 81.08) (end 156.34 93.48) (width 0.2) (layer "F.Cu") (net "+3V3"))
 (segment (start 156.34 93.48) (end 156.34 97.5) (width 0.2) (layer "F.Cu") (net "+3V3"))
 (segment (start 156.34 98.1965) (end 156.34 97.5) (width 0.2) (layer "B.Cu") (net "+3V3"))
 (segment (start 154.986 89.754) (end 152.246 89.754) (width 0.2) (layer "F.Cu") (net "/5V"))
 (segment (start 152.246 89.754) (end 146.5 95.5) (width 0.2) (layer "F.Cu") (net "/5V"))
 (segment (start 168.74 76) (end 154.986 89.754) (width 0.2) (layer "F.Cu") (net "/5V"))
 (segment (start 141.5 97.96) (end 143.96 95.5) (width 0.2) (layer "F.Cu") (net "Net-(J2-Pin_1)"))
 (segment (start 141.5 110.225) (end 141.5 97.96) (width 0.2) (layer "F.Cu") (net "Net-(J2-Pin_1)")))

